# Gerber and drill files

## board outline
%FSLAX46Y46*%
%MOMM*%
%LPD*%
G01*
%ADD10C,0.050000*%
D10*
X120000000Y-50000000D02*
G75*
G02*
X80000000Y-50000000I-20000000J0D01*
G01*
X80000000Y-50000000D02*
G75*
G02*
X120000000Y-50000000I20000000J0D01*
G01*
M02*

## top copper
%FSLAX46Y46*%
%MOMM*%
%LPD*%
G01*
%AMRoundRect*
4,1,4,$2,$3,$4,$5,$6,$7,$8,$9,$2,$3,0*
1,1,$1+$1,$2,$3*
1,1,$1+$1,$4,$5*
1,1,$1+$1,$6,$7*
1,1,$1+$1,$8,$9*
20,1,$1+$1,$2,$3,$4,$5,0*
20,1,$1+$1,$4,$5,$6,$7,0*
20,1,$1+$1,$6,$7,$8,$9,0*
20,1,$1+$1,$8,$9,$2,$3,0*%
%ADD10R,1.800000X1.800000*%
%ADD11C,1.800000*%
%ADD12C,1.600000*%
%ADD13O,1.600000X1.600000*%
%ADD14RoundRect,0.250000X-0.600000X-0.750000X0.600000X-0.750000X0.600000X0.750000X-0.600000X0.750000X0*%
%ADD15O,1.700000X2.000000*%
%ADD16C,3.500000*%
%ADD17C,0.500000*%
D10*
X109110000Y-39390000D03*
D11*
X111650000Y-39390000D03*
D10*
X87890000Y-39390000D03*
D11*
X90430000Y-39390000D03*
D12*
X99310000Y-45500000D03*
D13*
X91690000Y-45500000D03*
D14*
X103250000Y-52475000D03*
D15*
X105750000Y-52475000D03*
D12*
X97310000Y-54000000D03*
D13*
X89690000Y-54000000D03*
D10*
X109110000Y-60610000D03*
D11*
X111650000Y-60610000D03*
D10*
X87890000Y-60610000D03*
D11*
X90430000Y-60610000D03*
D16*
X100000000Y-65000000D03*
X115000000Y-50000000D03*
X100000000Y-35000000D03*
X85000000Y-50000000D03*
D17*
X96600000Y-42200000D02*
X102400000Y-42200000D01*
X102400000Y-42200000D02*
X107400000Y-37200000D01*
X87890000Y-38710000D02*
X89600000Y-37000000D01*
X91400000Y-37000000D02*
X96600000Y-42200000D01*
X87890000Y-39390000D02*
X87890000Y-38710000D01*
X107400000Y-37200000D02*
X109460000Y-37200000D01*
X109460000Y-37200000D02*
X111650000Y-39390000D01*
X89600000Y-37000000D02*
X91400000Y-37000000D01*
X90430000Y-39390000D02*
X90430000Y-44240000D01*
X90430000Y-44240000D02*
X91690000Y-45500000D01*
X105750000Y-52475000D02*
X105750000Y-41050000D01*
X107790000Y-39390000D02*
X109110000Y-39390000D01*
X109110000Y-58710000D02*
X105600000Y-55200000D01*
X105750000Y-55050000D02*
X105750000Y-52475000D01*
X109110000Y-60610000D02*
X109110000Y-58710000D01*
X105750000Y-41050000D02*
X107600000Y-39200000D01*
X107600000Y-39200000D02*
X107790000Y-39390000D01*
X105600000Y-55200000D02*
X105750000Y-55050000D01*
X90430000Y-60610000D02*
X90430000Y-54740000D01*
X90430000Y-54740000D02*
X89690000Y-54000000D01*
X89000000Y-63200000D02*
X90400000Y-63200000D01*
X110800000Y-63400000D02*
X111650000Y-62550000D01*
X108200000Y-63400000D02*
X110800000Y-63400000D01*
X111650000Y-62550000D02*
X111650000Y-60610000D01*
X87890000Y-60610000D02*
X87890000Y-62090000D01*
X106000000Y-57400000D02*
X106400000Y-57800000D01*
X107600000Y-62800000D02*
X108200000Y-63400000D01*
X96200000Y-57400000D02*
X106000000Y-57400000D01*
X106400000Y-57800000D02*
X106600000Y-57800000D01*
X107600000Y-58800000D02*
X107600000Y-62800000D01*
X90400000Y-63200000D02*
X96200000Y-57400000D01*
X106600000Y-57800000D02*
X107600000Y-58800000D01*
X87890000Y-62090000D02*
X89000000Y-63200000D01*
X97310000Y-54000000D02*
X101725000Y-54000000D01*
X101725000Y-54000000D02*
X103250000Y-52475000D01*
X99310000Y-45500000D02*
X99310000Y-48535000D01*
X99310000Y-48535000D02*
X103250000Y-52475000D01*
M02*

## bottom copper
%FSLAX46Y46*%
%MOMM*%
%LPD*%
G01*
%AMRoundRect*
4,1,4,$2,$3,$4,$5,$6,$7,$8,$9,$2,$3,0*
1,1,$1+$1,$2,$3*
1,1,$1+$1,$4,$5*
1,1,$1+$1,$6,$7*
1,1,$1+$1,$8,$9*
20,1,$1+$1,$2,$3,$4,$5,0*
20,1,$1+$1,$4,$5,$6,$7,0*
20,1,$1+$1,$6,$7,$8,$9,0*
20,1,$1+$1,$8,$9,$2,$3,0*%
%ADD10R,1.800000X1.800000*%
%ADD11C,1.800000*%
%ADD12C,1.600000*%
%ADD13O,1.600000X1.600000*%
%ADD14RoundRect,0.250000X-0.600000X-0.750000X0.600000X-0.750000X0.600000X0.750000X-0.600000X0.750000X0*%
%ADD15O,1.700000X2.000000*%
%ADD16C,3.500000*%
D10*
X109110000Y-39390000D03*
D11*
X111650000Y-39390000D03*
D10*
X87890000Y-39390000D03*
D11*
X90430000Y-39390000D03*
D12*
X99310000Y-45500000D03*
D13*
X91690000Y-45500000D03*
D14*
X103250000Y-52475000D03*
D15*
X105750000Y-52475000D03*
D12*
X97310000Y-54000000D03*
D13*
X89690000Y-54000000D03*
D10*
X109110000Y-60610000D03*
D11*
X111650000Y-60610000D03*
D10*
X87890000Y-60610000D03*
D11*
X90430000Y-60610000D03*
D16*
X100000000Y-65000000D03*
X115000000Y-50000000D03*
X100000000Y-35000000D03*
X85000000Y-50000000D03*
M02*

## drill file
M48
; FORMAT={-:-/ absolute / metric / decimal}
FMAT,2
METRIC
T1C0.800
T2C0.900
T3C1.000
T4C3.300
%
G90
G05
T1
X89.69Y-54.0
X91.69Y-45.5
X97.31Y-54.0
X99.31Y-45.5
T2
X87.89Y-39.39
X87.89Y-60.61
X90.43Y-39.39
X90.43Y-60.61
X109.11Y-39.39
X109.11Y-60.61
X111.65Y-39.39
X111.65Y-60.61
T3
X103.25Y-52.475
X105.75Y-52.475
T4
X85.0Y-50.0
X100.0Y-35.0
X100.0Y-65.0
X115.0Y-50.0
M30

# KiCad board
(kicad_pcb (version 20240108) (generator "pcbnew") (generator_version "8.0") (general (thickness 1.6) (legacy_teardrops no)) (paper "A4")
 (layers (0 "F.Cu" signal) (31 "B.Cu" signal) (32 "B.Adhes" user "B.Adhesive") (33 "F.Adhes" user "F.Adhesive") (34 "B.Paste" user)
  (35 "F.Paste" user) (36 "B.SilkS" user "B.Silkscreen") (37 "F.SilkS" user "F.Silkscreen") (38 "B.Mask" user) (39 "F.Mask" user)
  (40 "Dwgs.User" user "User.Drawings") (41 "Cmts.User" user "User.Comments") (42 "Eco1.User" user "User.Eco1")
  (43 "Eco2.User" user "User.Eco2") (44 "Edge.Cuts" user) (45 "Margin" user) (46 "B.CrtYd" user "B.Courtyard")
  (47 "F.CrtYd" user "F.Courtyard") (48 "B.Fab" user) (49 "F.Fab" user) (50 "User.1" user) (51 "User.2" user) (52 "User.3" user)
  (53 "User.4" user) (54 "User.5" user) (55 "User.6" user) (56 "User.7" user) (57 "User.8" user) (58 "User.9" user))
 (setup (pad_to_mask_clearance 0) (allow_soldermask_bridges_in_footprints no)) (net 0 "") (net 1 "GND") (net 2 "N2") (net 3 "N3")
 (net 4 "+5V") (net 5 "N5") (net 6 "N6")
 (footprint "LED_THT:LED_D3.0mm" (layer "F.Cu") (at 109.11 39.39)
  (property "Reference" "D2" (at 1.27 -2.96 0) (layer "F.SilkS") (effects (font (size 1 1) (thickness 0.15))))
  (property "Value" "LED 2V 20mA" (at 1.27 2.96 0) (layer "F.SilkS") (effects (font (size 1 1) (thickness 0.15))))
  (pad "1" thru_hole rect (at 0 0) (size 1.8 1.8) (drill 0.9) (layers "*.Cu" "*.Mask") (remove_unused_layers no) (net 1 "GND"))
  (pad "2" thru_hole circle (at 2.54 0) (size 1.8 1.8) (drill 0.9) (layers "*.Cu" "*.Mask") (remove_unused_layers no) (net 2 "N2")))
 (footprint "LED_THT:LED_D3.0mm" (layer "F.Cu") (at 87.89 39.39)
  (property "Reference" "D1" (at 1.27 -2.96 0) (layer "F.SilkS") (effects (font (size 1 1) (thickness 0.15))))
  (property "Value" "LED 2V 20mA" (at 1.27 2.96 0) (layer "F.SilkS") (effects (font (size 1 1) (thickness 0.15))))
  (pad "1" thru_hole rect (at 0 0) (size 1.8 1.8) (drill 0.9) (layers "*.Cu" "*.Mask") (remove_unused_layers no) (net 2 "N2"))
  (pad "2" thru_hole circle (at 2.54 0) (size 1.8 1.8) (drill 0.9) (layers "*.Cu" "*.Mask") (remove_unused_layers no) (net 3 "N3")))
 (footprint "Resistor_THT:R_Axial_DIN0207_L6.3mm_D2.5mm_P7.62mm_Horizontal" (layer "F.Cu") (at 99.31 45.5 180)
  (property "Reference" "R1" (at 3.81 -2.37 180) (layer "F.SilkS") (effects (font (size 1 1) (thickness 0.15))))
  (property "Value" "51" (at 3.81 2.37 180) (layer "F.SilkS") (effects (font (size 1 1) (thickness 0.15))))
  (pad "1" thru_hole circle (at 0 0 180) (size 1.6 1.6) (drill 0.8) (layers "*.Cu" "*.Mask") (remove_unused_layers no) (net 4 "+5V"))
  (pad "2" thru_hole oval (at 7.62 0 180) (size 1.6 1.6) (drill 0.8) (layers "*.Cu" "*.Mask") (remove_unused_layers no) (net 3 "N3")))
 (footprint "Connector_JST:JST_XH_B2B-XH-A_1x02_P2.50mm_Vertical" (layer "F.Cu") (at 103.25 52.475)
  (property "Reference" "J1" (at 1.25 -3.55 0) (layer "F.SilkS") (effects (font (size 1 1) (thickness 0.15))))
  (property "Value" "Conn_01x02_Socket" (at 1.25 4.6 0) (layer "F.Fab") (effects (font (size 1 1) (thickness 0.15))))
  (pad "1" thru_hole roundrect (at 0 0) (size 1.7 2) (drill 1) (layers "*.Cu" "*.Mask") (remove_unused_layers no)
   (roundrect_rratio 0.147059) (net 4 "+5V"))
  (pad "2" thru_hole oval (at 2.5 0) (size 1.7 2) (drill 1) (layers "*.Cu" "*.Mask") (remove_unused_layers no) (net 1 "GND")))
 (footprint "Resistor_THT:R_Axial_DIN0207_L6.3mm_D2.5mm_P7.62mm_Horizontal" (layer "F.Cu") (at 97.31 54 180)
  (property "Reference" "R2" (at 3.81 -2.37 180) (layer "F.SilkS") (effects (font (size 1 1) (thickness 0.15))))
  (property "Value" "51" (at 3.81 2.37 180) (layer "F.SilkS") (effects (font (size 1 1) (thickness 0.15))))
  (pad "1" thru_hole circle (at 0 0 180) (size 1.6 1.6) (drill 0.8) (layers "*.Cu" "*.Mask") (remove_unused_layers no) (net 4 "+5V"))
  (pad "2" thru_hole oval (at 7.62 0 180) (size 1.6 1.6) (drill 0.8) (layers "*.Cu" "*.Mask") (remove_unused_layers no) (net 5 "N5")))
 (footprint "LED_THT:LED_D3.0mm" (layer "F.Cu") (at 109.11 60.61)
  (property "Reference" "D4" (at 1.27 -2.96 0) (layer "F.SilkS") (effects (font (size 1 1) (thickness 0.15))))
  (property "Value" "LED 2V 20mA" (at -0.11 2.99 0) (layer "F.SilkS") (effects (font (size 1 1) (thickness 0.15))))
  (pad "1" thru_hole rect (at 0 0) (size 1.8 1.8) (drill 0.9) (layers "*.Cu" "*.Mask") (remove_unused_layers no) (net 1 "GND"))
  (pad "2" thru_hole circle (at 2.54 0) (size 1.8 1.8) (drill 0.9) (layers "*.Cu" "*.Mask") (remove_unused_layers no) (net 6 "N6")))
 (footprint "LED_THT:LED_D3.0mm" (layer "F.Cu") (at 87.89 60.61)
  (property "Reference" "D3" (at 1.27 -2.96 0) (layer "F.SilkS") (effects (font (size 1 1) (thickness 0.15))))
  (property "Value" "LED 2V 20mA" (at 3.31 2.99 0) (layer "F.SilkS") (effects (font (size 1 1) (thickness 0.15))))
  (pad "1" thru_hole rect (at 0 0) (size 1.8 1.8) (drill 0.9) (layers "*.Cu" "*.Mask") (remove_unused_layers no) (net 6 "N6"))
  (pad "2" thru_hole circle (at 2.54 0) (size 1.8 1.8) (drill 0.9) (layers "*.Cu" "*.Mask") (remove_unused_layers no) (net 5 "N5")))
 (gr_circle (center 100 50) (end 120 50) (stroke (width 0.05) (type default)) (fill none) (layer "Edge.Cuts"))
 (via (at 100 65) (size 3.5) (drill 3.3) (layers "F.Cu" "B.Cu") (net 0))
 (via (at 115 50) (size 3.5) (drill 3.3) (layers "F.Cu" "B.Cu") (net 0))
 (via (at 100 35) (size 3.5) (drill 3.3) (layers "F.Cu" "B.Cu") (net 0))
 (via (at 85 50) (size 3.5) (drill 3.3) (layers "F.Cu" "B.Cu") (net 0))
 (segment (start 96.6 42.2) (end 102.4 42.2) (width 0.5) (layer "F.Cu") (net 2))
 (segment (start 102.4 42.2) (end 107.4 37.2) (width 0.5) (layer "F.Cu") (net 2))
 (segment (start 87.89 38.71) (end 89.6 37) (width 0.5) (layer "F.Cu") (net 2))
 (segment (start 91.4 37) (end 96.6 42.2) (width 0.5) (layer "F.Cu") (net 2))
 (segment (start 87.89 39.39) (end 87.89 38.71) (width 0.5) (layer "F.Cu") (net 2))
 (segment (start 107.4 37.2) (end 109.46 37.2) (width 0.5) (layer "F.Cu") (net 2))
 (segment (start 109.46 37.2) (end 111.65 39.39) (width 0.5) (layer "F.Cu") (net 2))
 (segment (start 89.6 37) (end 91.4 37) (width 0.5) (layer "F.Cu") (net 2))
 (segment (start 90.43 39.39) (end 90.43 44.24) (width 0.5) (layer "F.Cu") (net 3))
 (segment (start 90.43 44.24) (end 91.69 45.5) (width 0.5) (layer "F.Cu") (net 3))
 (segment (start 105.75 52.475) (end 105.75 41.05) (width 0.5) (layer "F.Cu") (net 1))
 (segment (start 107.79 39.39) (end 109.11 39.39) (width 0.5) (layer "F.Cu") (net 1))
 (segment (start 109.11 58.71) (end 105.6 55.2) (width 0.5) (layer "F.Cu") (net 1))
 (segment (start 105.75 55.05) (end 105.75 52.475) (width 0.5) (layer "F.Cu") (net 1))
 (segment (start 109.11 60.61) (end 109.11 58.71) (width 0.5) (layer "F.Cu") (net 1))
 (segment (start 105.75 41.05) (end 107.6 39.2) (width 0.5) (layer "F.Cu") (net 1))
 (segment (start 107.6 39.2) (end 107.79 39.39) (width 0.5) (layer "F.Cu") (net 1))
 (segment (start 105.6 55.2) (end 105.75 55.05) (width 0.5) (layer "F.Cu") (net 1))
 (segment (start 90.43 60.61) (end 90.43 54.74) (width 0.5) (layer "F.Cu") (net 5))
 (segment (start 90.43 54.74) (end 89.69 54) (width 0.5) (layer "F.Cu") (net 5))
 (segment (start 89 63.2) (end 90.4 63.2) (width 0.5) (layer "F.Cu") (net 6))
 (segment (start 110.8 63.4) (end 111.65 62.55) (width 0.5) (layer "F.Cu") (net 6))
 (segment (start 108.2 63.4) (end 110.8 63.4) (width 0.5) (layer "F.Cu") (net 6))
 (segment (start 111.65 62.55) (end 111.65 60.61) (width 0.5) (layer "F.Cu") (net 6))
 (segment (start 87.89 60.61) (end 87.89 62.09) (width 0.5) (layer "F.Cu") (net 6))
 (segment (start 106 57.4) (end 106.4 57.8) (width 0.5) (layer "F.Cu") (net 6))
 (segment (start 107.6 62.8) (end 108.2 63.4) (width 0.5) (layer "F.Cu") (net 6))
 (segment (start 96.2 57.4) (end 106 57.4) (width 0.5) (layer "F.Cu") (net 6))
 (segment (start 106.4 57.8) (end 106.6 57.8) (width 0.5) (layer "F.Cu") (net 6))
 (segment (start 107.6 58.8) (end 107.6 62.8) (width 0.5) (layer "F.Cu") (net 6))
 (segment (start 90.4 63.2) (end 96.2 57.4) (width 0.5) (layer "F.Cu") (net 6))
 (segment (start 106.6 57.8) (end 107.6 58.8) (width 0.5) (layer "F.Cu") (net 6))
 (segment (start 87.89 62.09) (end 89 63.2) (width 0.5) (layer "F.Cu") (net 6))
 (segment (start 97.31 54) (end 101.725 54) (width 0.5) (layer "F.Cu") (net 4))
 (segment (start 101.725 54) (end 103.25 52.475) (width 0.5) (layer "F.Cu") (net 4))
 (segment (start 99.31 45.5) (end 99.31 48.535) (width 0.5) (layer "F.Cu") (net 4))
 (segment (start 99.31 48.535) (end 103.25 52.475) (width 0.5) (layer "F.Cu") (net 4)))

